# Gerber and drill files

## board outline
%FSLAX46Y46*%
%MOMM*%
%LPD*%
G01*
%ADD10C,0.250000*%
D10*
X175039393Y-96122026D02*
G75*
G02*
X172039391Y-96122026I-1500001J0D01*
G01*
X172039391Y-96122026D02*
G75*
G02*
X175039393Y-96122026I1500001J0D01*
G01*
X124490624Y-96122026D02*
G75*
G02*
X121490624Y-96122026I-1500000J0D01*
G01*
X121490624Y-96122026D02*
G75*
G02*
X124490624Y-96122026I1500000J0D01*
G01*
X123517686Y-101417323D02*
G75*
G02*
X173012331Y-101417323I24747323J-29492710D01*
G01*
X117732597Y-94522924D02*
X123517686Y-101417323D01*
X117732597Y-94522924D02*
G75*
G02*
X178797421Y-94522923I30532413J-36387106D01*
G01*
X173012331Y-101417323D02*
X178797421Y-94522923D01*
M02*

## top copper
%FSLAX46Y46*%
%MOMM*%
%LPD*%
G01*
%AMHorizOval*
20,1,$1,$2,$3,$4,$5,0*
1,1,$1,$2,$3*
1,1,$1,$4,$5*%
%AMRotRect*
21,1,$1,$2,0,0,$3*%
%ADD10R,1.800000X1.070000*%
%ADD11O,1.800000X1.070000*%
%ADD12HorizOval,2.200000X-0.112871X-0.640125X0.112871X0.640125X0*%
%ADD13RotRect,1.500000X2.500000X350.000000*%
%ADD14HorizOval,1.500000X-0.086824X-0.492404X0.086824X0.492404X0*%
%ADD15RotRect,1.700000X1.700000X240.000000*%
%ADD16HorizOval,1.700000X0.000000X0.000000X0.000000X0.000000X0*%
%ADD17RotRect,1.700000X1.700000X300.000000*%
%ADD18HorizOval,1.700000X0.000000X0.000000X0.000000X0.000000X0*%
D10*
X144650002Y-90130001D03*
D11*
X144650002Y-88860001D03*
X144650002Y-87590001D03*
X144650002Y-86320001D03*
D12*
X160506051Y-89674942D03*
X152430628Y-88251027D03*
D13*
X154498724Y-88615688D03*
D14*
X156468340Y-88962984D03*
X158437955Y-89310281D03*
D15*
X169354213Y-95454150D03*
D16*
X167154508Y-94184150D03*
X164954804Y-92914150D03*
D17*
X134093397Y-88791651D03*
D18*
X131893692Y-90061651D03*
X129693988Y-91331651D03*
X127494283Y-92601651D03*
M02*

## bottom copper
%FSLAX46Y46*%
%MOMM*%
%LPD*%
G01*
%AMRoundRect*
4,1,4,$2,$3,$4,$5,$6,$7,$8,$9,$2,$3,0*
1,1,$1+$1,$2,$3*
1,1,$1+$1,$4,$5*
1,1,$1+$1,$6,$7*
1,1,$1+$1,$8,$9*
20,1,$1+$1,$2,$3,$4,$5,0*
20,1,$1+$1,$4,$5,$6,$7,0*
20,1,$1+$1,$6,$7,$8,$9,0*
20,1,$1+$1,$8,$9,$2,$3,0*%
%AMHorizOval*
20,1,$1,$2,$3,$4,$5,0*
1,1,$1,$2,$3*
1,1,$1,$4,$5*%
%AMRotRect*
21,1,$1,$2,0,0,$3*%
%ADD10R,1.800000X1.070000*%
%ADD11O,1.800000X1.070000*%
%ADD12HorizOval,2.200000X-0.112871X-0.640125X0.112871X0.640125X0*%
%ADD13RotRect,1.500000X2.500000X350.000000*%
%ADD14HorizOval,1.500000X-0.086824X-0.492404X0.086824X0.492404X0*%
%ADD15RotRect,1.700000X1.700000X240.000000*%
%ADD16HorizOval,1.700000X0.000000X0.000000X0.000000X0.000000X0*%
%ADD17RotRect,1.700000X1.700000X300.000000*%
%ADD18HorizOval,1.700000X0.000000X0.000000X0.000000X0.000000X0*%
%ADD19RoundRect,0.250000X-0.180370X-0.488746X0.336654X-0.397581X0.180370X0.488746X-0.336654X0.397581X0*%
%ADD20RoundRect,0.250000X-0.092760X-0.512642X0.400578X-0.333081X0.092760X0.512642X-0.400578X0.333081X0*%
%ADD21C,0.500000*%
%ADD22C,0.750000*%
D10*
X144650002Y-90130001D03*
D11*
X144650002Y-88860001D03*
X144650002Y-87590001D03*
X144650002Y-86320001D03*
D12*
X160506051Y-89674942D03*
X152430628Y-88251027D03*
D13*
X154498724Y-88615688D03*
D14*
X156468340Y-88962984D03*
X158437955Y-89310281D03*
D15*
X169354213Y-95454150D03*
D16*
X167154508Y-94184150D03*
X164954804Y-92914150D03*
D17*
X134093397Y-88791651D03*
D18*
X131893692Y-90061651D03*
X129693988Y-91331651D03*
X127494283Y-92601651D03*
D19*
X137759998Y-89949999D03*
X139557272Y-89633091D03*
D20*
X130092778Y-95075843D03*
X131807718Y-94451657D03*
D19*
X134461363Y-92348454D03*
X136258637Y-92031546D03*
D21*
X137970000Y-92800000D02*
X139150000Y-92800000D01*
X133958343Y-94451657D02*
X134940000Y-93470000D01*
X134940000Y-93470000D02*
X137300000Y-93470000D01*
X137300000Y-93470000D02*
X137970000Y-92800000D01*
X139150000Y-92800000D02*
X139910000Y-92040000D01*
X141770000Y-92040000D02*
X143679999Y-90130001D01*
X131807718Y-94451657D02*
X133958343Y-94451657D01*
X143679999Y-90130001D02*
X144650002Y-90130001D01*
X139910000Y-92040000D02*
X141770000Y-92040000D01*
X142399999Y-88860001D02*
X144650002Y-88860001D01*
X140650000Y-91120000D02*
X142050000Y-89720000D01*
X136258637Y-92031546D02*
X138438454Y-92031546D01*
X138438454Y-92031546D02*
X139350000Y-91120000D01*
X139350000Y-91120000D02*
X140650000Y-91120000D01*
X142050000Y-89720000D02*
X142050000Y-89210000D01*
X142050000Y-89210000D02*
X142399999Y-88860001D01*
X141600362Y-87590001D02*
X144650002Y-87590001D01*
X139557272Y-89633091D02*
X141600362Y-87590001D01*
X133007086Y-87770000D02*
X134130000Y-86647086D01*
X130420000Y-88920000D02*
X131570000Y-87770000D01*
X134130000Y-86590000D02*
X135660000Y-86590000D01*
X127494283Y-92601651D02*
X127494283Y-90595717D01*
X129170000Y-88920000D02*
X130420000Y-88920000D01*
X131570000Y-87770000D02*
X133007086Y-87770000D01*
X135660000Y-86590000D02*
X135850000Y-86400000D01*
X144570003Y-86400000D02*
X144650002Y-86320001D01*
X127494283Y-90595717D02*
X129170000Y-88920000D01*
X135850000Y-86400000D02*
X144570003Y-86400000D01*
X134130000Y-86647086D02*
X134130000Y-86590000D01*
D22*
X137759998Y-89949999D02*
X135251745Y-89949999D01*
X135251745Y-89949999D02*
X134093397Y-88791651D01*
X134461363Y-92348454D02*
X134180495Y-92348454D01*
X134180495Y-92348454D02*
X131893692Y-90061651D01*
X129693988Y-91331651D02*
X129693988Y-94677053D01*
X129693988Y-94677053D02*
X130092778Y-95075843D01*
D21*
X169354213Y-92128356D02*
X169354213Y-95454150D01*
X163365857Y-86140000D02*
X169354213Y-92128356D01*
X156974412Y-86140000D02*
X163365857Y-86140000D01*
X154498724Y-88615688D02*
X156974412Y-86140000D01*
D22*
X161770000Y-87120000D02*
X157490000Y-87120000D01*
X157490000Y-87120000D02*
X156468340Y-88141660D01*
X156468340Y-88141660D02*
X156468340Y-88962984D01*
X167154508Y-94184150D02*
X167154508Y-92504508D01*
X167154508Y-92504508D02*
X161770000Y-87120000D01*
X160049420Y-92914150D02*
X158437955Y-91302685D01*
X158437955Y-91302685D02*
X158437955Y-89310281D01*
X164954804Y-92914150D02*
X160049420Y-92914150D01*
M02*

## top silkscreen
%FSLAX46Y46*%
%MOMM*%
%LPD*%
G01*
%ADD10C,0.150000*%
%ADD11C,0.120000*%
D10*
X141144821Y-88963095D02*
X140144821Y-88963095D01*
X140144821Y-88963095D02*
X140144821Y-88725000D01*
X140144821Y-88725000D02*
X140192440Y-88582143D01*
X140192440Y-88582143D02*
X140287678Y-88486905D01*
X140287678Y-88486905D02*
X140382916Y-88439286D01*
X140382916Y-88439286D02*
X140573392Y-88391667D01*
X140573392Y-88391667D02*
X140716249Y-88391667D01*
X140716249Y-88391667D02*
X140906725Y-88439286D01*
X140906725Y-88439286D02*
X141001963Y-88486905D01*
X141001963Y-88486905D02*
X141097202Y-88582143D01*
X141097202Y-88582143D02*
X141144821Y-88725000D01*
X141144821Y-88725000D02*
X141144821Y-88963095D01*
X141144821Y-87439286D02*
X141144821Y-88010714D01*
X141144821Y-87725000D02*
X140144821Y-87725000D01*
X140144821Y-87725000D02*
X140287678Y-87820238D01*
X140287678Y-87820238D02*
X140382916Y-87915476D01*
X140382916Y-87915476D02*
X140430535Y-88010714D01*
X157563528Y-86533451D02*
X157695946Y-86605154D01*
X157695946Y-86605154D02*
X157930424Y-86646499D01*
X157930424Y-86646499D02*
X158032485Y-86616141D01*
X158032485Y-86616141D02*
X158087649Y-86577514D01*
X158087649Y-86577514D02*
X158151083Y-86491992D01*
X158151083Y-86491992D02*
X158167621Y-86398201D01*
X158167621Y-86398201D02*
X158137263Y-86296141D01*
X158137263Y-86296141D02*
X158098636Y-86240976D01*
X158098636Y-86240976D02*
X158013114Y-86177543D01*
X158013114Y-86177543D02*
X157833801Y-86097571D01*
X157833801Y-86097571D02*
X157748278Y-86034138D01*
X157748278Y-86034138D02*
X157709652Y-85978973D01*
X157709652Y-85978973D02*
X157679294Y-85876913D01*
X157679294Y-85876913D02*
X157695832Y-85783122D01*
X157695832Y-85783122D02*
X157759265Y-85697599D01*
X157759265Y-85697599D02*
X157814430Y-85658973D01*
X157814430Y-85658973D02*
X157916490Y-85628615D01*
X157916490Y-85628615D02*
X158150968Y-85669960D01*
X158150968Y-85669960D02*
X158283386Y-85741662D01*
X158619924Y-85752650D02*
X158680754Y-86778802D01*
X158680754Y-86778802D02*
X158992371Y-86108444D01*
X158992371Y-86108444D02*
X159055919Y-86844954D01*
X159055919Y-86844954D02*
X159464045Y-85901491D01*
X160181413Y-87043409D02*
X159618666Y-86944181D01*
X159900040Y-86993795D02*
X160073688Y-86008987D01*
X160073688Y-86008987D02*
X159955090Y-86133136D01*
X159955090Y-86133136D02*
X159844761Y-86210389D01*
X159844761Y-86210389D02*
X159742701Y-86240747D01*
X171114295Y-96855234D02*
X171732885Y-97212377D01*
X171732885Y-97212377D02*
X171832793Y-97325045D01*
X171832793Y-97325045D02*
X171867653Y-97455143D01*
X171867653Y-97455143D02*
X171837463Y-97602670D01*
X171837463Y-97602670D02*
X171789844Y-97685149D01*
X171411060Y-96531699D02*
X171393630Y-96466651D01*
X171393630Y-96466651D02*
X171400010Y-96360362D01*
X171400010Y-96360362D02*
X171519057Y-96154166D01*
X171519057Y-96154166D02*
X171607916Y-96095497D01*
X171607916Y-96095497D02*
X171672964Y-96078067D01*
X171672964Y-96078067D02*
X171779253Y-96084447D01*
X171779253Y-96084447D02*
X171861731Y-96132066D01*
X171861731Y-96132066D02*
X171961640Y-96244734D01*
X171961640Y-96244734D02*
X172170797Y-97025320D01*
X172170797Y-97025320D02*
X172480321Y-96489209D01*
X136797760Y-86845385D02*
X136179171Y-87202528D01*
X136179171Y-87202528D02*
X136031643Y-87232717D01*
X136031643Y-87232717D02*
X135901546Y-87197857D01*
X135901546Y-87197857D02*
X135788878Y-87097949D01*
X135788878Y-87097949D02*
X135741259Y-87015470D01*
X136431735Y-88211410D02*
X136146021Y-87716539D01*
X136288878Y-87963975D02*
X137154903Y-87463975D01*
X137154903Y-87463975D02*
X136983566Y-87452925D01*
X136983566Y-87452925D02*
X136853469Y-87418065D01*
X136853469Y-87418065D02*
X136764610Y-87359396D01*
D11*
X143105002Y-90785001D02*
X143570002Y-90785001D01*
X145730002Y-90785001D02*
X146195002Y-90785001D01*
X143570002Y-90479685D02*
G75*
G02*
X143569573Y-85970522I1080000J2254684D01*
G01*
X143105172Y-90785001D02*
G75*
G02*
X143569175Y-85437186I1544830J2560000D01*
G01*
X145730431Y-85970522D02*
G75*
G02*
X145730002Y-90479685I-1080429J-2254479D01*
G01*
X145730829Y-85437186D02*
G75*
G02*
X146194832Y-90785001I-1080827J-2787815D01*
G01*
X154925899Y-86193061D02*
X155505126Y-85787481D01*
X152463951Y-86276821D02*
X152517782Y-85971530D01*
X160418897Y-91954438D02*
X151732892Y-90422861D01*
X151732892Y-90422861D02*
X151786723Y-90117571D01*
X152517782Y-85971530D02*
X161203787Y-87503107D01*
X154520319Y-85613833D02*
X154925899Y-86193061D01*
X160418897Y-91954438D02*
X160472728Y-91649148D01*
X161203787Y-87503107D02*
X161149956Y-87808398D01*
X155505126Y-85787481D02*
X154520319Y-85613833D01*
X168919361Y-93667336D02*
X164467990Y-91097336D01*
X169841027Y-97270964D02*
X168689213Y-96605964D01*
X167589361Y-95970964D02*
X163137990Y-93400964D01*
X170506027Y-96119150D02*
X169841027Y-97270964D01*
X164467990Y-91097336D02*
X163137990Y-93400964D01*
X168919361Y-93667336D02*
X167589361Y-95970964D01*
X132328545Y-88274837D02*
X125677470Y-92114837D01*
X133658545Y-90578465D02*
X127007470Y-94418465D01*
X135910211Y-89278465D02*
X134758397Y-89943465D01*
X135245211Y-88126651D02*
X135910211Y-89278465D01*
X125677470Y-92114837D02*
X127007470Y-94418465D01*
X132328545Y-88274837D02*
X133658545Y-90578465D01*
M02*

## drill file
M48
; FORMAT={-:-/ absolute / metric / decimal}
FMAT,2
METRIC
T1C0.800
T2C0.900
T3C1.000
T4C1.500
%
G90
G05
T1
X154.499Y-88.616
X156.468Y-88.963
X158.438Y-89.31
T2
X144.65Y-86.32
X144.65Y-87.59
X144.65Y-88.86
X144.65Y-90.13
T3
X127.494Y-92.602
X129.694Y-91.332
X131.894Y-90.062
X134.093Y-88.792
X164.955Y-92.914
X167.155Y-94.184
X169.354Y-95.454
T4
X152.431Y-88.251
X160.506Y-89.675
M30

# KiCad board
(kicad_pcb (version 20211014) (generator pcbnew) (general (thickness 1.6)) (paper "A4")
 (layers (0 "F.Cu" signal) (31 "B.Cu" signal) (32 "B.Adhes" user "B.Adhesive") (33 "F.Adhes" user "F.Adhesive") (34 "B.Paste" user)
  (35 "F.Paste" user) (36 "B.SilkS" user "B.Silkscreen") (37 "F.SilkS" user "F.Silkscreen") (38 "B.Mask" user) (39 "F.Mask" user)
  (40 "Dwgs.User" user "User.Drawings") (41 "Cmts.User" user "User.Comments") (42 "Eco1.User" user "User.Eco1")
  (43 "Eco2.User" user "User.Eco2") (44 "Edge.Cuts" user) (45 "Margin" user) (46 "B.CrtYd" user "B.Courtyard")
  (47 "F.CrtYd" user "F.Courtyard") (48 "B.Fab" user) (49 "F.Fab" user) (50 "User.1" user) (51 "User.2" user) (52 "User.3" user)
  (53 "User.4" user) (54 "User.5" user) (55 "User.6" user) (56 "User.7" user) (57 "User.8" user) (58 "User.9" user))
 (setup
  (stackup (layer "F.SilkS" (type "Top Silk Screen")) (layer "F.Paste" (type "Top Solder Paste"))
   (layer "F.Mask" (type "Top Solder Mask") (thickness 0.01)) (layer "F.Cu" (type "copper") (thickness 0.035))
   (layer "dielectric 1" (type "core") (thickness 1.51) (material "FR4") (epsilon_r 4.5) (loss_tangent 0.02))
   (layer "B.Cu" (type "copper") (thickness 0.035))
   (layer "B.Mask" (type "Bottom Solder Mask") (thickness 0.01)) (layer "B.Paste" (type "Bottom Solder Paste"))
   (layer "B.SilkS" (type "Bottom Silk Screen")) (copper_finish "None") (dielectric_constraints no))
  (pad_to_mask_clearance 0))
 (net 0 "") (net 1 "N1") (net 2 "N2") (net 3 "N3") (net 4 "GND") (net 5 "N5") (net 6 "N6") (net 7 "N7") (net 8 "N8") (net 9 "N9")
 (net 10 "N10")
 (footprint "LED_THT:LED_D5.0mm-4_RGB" (layer "F.Cu") (at 144.650002 90.130001 90)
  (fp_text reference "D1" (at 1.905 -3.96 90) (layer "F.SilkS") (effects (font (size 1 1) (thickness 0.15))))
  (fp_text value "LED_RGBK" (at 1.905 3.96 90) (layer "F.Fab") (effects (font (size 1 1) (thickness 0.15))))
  (fp_line (start -0.655 -1.545) (end -0.655 -1.08) (layer "F.SilkS") (width 0.12))
  (fp_line (start -0.655 1.08) (end -0.655 1.545) (layer "F.SilkS") (width 0.12))
  (fp_arc (start -0.349684 -1.08) (mid 1.904762 -2.5) (end 4.159479 -1.080429) (layer "F.SilkS") (width 0.12))
  (fp_arc (start -0.655 -1.54483) (mid 2.163456 -2.978809) (end 4.692815 -1.080827) (layer "F.SilkS") (width 0.12))
  (fp_arc (start 4.159479 1.080429) (mid 1.904762 2.5) (end -0.349684 1.08) (layer "F.SilkS") (width 0.12))
  (fp_arc (start 4.692815 1.080827) (mid 2.163456 2.978808) (end -0.655 1.54483) (layer "F.SilkS") (width 0.12))
  (pad "1" thru_hole rect locked (at 0 0 90) (size 1.07 1.8) (drill 0.9) (layers *.Cu *.Mask) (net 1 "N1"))
  (pad "2" thru_hole oval locked (at 1.27 0 90) (size 1.07 1.8) (drill 0.9) (layers *.Cu *.Mask) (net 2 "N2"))
  (pad "3" thru_hole oval locked (at 2.54 0 90) (size 1.07 1.8) (drill 0.9) (layers *.Cu *.Mask) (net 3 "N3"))
  (pad "4" thru_hole oval locked (at 3.81 0 90) (size 1.07 1.8) (drill 0.9) (layers *.Cu *.Mask) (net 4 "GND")))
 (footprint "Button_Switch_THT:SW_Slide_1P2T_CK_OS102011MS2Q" (layer "F.Cu") (at 154.498724 88.615688 -10)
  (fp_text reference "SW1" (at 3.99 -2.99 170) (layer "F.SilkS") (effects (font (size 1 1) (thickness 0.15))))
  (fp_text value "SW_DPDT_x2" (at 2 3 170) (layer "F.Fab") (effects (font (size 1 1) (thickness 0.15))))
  (fp_line (start 0 -2.46) (end 0.5 -2.96) (layer "F.SilkS") (width 0.12))
  (fp_line (start -2.41 -1.95) (end -2.41 -2.26) (layer "F.SilkS") (width 0.12))
  (fp_line (start 6.41 2.26) (end -2.41 2.26) (layer "F.SilkS") (width 0.12))
  (fp_line (start -2.41 2.26) (end -2.41 1.95) (layer "F.SilkS") (width 0.12))
  (fp_line (start -2.41 -2.26) (end 6.41 -2.26) (layer "F.SilkS") (width 0.12))
  (fp_line (start -0.5 -2.96) (end 0 -2.46) (layer "F.SilkS") (width 0.12))
  (fp_line (start 6.41 2.26) (end 6.41 1.95) (layer "F.SilkS") (width 0.12))
  (fp_line (start 6.41 -2.26) (end 6.41 -1.95) (layer "F.SilkS") (width 0.12))
  (fp_line (start 0.5 -2.96) (end -0.5 -2.96) (layer "F.SilkS") (width 0.12))
  (pad "" thru_hole oval locked (at 6.1 0 350) (size 2.2 3.5) (drill 1.5) (layers *.Cu *.Mask))
  (pad "" thru_hole oval locked (at -2.1 0 350) (size 2.2 3.5) (drill 1.5) (layers *.Cu *.Mask))
  (pad "1" thru_hole rect locked (at 0 0 350) (size 1.5 2.5) (drill 0.8) (layers *.Cu *.Mask) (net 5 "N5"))
  (pad "2" thru_hole oval locked (at 2 0 350) (size 1.5 2.5) (drill 0.8) (layers *.Cu *.Mask) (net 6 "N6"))
  (pad "3" thru_hole oval locked (at 4 0 350) (size 1.5 2.5) (drill 0.8) (layers *.Cu *.Mask) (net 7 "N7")))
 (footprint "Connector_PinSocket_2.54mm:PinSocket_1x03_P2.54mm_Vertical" (layer "F.Cu") (at 169.354213 95.45415 -120)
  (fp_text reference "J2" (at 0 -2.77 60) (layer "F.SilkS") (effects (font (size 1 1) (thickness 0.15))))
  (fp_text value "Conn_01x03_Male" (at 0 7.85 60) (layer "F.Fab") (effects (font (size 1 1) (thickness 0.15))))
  (fp_line (start -1.33 1.27) (end -1.33 6.41) (layer "F.SilkS") (width 0.12))
  (fp_line (start 1.33 -1.33) (end 1.33 0) (layer "F.SilkS") (width 0.12))
  (fp_line (start 1.33 1.27) (end 1.33 6.41) (layer "F.SilkS") (width 0.12))
  (fp_line (start 0 -1.33) (end 1.33 -1.33) (layer "F.SilkS") (width 0.12))
  (fp_line (start -1.33 6.41) (end 1.33 6.41) (layer "F.SilkS") (width 0.12))
  (fp_line (start -1.33 1.27) (end 1.33 1.27) (layer "F.SilkS") (width 0.12))
  (pad "1" thru_hole rect locked (at 0 0 240) (size 1.7 1.7) (drill 1) (layers *.Cu *.Mask) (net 5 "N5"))
  (pad "2" thru_hole oval locked (at 0 2.54 240) (size 1.7 1.7) (drill 1) (layers *.Cu *.Mask) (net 6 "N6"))
  (pad "3" thru_hole oval locked (at 0 5.08 240) (size 1.7 1.7) (drill 1) (layers *.Cu *.Mask) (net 7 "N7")))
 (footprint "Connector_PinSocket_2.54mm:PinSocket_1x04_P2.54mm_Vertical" (layer "F.Cu") (at 134.093397 88.791651 -60)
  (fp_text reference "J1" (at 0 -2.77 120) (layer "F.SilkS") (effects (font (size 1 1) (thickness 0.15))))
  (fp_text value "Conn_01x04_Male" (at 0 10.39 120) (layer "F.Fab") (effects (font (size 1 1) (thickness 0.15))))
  (fp_line (start -1.33 1.27) (end -1.33 8.95) (layer "F.SilkS") (width 0.12))
  (fp_line (start 1.33 1.27) (end 1.33 8.95) (layer "F.SilkS") (width 0.12))
  (fp_line (start 1.33 -1.33) (end 1.33 0) (layer "F.SilkS") (width 0.12))
  (fp_line (start 0 -1.33) (end 1.33 -1.33) (layer "F.SilkS") (width 0.12))
  (fp_line (start -1.33 8.95) (end 1.33 8.95) (layer "F.SilkS") (width 0.12))
  (fp_line (start -1.33 1.27) (end 1.33 1.27) (layer "F.SilkS") (width 0.12))
  (pad "1" thru_hole rect locked (at 0 0 300) (size 1.7 1.7) (drill 1) (layers *.Cu *.Mask) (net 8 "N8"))
  (pad "2" thru_hole oval locked (at 0 2.54 300) (size 1.7 1.7) (drill 1) (layers *.Cu *.Mask) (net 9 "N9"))
  (pad "3" thru_hole oval locked (at 0 5.08 300) (size 1.7 1.7) (drill 1) (layers *.Cu *.Mask) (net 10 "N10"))
  (pad "4" thru_hole oval locked (at 0 7.62 300) (size 1.7 1.7) (drill 1) (layers *.Cu *.Mask) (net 4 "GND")))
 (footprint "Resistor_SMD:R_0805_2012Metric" (layer "B.Cu") (at 138.658635 89.791545 10)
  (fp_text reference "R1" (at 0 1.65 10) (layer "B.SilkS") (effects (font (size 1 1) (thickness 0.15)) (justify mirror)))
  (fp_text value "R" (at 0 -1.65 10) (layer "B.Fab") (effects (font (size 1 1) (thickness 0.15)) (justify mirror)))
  (pad "1" smd roundrect locked (at -0.9125 0 10) (size 1.025 1.4) (layers "B.Cu" "B.Paste" "B.Mask") (roundrect_rratio 0.243902)
   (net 8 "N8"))
  (pad "2" smd roundrect locked (at 0.9125 0 10) (size 1.025 1.4) (layers "B.Cu" "B.Paste" "B.Mask") (roundrect_rratio 0.243902)
   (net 3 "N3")))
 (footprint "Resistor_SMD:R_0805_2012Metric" (layer "B.Cu") (at 130.950248 94.76375 20)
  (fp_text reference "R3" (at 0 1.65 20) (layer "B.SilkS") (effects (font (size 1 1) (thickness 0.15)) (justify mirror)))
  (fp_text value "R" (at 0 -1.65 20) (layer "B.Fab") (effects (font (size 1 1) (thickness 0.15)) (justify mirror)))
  (pad "1" smd roundrect locked (at -0.9125 0 20) (size 1.025 1.4) (layers "B.Cu" "B.Paste" "B.Mask") (roundrect_rratio 0.243902)
   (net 10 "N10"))
  (pad "2" smd roundrect locked (at 0.9125 0 20) (size 1.025 1.4) (layers "B.Cu" "B.Paste" "B.Mask") (roundrect_rratio 0.243902)
   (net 1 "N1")))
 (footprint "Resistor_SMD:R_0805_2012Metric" (layer "B.Cu") (at 135.36 92.19 10)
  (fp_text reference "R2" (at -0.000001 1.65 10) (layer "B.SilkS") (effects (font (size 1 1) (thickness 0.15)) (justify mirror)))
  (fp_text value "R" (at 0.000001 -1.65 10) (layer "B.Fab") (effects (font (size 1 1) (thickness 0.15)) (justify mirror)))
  (pad "1" smd roundrect locked (at -0.9125 0 10) (size 1.025 1.4) (layers "B.Cu" "B.Paste" "B.Mask") (roundrect_rratio 0.243902)
   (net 9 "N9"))
  (pad "2" smd roundrect locked (at 0.9125 0 10) (size 1.025 1.4) (layers "B.Cu" "B.Paste" "B.Mask") (roundrect_rratio 0.243902)
   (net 2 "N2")))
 (gr_circle (center 173.539392 96.122026) (end 174.503573 94.972958) (layer "Edge.Cuts") (width 0.25) (fill none))
 (gr_circle (center 122.990624 96.122026) (end 123.954806 94.97296) (layer "Edge.Cuts") (width 0.25) (fill none))
 (gr_arc (start 123.517686 101.417323) (mid 148.265009 92.410034) (end 173.012331 101.417323) (layer "Edge.Cuts") (width 0.25))
 (gr_line (start 117.732597 94.522924) (end 123.517686 101.417323) (layer "Edge.Cuts") (width 0.25))
 (gr_arc (start 117.732597 94.522924) (mid 148.265009 83.410034) (end 178.797421 94.522923) (layer "Edge.Cuts") (width 0.25))
 (gr_line (start 173.012331 101.417323) (end 178.797421 94.522923) (layer "Edge.Cuts") (width 0.25))
 (segment (start 137.97 92.8) (end 139.15 92.8) (width 0.5) (layer "B.Cu") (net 1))
 (segment (start 133.958343 94.451657) (end 134.94 93.47) (width 0.5) (layer "B.Cu") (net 1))
 (segment (start 134.94 93.47) (end 137.3 93.47) (width 0.5) (layer "B.Cu") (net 1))
 (segment (start 137.3 93.47) (end 137.97 92.8) (width 0.5) (layer "B.Cu") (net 1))
 (segment (start 139.15 92.8) (end 139.91 92.04) (width 0.5) (layer "B.Cu") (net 1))
 (segment (start 141.77 92.04) (end 143.679999 90.130001) (width 0.5) (layer "B.Cu") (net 1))
 (segment (start 131.807718 94.451657) (end 133.958343 94.451657) (width 0.5) (layer "B.Cu") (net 1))
 (segment (start 143.679999 90.130001) (end 144.650002 90.130001) (width 0.5) (layer "B.Cu") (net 1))
 (segment (start 139.91 92.04) (end 141.77 92.04) (width 0.5) (layer "B.Cu") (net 1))
 (segment (start 142.399999 88.860001) (end 144.650002 88.860001) (width 0.5) (layer "B.Cu") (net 2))
 (segment (start 140.65 91.12) (end 142.05 89.72) (width 0.5) (layer "B.Cu") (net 2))
 (segment (start 136.258637 92.031546) (end 138.438454 92.031546) (width 0.5) (layer "B.Cu") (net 2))
 (segment (start 138.438454 92.031546) (end 139.35 91.12) (width 0.5) (layer "B.Cu") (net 2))
 (segment (start 139.35 91.12) (end 140.65 91.12) (width 0.5) (layer "B.Cu") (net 2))
 (segment (start 142.05 89.72) (end 142.05 89.21) (width 0.5) (layer "B.Cu") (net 2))
 (segment (start 142.05 89.21) (end 142.399999 88.860001) (width 0.5) (layer "B.Cu") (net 2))
 (segment (start 141.600362 87.590001) (end 144.650002 87.590001) (width 0.5) (layer "B.Cu") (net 3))
 (segment (start 139.557272 89.633091) (end 141.600362 87.590001) (width 0.5) (layer "B.Cu") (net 3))
 (segment (start 133.007086 87.77) (end 134.13 86.647086) (width 0.5) (layer "B.Cu") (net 4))
 (segment (start 130.42 88.92) (end 131.57 87.77) (width 0.5) (layer "B.Cu") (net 4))
 (segment (start 134.13 86.59) (end 135.66 86.59) (width 0.5) (layer "B.Cu") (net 4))
 (segment (start 127.494283 92.601651) (end 127.494283 90.595717) (width 0.5) (layer "B.Cu") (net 4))
 (segment (start 129.17 88.92) (end 130.42 88.92) (width 0.5) (layer "B.Cu") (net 4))
 (segment (start 131.57 87.77) (end 133.007086 87.77) (width 0.5) (layer "B.Cu") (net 4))
 (segment (start 135.66 86.59) (end 135.85 86.4) (width 0.5) (layer "B.Cu") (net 4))
 (segment (start 144.570003 86.4) (end 144.650002 86.320001) (width 0.5) (layer "B.Cu") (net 4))
 (segment (start 127.494283 90.595717) (end 129.17 88.92) (width 0.5) (layer "B.Cu") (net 4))
 (segment (start 135.85 86.4) (end 144.570003 86.4) (width 0.5) (layer "B.Cu") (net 4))
 (segment (start 134.13 86.647086) (end 134.13 86.59) (width 0.5) (layer "B.Cu") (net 4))
 (segment (start 137.759998 89.949999) (end 135.251745 89.949999) (width 0.75) (layer "B.Cu") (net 8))
 (segment (start 135.251745 89.949999) (end 134.093397 88.791651) (width 0.75) (layer "B.Cu") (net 8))
 (segment (start 134.461363 92.348454) (end 134.180495 92.348454) (width 0.75) (layer "B.Cu") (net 9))
 (segment (start 134.180495 92.348454) (end 131.893692 90.061651) (width 0.75) (layer "B.Cu") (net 9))
 (segment (start 129.693988 91.331651) (end 129.693988 94.677053) (width 0.75) (layer "B.Cu") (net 10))
 (segment (start 129.693988 94.677053) (end 130.092778 95.075843) (width 0.75) (layer "B.Cu") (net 10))
 (segment (start 169.354213 92.128356) (end 169.354213 95.45415) (width 0.5) (layer "B.Cu") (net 5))
 (segment (start 163.365857 86.14) (end 169.354213 92.128356) (width 0.5) (layer "B.Cu") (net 5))
 (segment (start 156.974412 86.14) (end 163.365857 86.14) (width 0.5) (layer "B.Cu") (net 5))
 (segment (start 154.498724 88.615688) (end 156.974412 86.14) (width 0.5) (layer "B.Cu") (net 5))
 (segment (start 161.77 87.12) (end 157.49 87.12) (width 0.75) (layer "B.Cu") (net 6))
 (segment (start 157.49 87.12) (end 156.46834 88.14166) (width 0.75) (layer "B.Cu") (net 6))
 (segment (start 156.46834 88.14166) (end 156.46834 88.962984) (width 0.75) (layer "B.Cu") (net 6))
 (segment (start 167.154508 94.18415) (end 167.154508 92.504508) (width 0.75) (layer "B.Cu") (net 6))
 (segment (start 167.154508 92.504508) (end 161.77 87.12) (width 0.75) (layer "B.Cu") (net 6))
 (segment (start 160.04942 92.91415) (end 158.437955 91.302685) (width 0.75) (layer "B.Cu") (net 7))
 (segment (start 158.437955 91.302685) (end 158.437955 89.310281) (width 0.75) (layer "B.Cu") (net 7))
 (segment (start 164.954804 92.91415) (end 160.04942 92.91415) (width 0.75) (layer "B.Cu") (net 7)))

